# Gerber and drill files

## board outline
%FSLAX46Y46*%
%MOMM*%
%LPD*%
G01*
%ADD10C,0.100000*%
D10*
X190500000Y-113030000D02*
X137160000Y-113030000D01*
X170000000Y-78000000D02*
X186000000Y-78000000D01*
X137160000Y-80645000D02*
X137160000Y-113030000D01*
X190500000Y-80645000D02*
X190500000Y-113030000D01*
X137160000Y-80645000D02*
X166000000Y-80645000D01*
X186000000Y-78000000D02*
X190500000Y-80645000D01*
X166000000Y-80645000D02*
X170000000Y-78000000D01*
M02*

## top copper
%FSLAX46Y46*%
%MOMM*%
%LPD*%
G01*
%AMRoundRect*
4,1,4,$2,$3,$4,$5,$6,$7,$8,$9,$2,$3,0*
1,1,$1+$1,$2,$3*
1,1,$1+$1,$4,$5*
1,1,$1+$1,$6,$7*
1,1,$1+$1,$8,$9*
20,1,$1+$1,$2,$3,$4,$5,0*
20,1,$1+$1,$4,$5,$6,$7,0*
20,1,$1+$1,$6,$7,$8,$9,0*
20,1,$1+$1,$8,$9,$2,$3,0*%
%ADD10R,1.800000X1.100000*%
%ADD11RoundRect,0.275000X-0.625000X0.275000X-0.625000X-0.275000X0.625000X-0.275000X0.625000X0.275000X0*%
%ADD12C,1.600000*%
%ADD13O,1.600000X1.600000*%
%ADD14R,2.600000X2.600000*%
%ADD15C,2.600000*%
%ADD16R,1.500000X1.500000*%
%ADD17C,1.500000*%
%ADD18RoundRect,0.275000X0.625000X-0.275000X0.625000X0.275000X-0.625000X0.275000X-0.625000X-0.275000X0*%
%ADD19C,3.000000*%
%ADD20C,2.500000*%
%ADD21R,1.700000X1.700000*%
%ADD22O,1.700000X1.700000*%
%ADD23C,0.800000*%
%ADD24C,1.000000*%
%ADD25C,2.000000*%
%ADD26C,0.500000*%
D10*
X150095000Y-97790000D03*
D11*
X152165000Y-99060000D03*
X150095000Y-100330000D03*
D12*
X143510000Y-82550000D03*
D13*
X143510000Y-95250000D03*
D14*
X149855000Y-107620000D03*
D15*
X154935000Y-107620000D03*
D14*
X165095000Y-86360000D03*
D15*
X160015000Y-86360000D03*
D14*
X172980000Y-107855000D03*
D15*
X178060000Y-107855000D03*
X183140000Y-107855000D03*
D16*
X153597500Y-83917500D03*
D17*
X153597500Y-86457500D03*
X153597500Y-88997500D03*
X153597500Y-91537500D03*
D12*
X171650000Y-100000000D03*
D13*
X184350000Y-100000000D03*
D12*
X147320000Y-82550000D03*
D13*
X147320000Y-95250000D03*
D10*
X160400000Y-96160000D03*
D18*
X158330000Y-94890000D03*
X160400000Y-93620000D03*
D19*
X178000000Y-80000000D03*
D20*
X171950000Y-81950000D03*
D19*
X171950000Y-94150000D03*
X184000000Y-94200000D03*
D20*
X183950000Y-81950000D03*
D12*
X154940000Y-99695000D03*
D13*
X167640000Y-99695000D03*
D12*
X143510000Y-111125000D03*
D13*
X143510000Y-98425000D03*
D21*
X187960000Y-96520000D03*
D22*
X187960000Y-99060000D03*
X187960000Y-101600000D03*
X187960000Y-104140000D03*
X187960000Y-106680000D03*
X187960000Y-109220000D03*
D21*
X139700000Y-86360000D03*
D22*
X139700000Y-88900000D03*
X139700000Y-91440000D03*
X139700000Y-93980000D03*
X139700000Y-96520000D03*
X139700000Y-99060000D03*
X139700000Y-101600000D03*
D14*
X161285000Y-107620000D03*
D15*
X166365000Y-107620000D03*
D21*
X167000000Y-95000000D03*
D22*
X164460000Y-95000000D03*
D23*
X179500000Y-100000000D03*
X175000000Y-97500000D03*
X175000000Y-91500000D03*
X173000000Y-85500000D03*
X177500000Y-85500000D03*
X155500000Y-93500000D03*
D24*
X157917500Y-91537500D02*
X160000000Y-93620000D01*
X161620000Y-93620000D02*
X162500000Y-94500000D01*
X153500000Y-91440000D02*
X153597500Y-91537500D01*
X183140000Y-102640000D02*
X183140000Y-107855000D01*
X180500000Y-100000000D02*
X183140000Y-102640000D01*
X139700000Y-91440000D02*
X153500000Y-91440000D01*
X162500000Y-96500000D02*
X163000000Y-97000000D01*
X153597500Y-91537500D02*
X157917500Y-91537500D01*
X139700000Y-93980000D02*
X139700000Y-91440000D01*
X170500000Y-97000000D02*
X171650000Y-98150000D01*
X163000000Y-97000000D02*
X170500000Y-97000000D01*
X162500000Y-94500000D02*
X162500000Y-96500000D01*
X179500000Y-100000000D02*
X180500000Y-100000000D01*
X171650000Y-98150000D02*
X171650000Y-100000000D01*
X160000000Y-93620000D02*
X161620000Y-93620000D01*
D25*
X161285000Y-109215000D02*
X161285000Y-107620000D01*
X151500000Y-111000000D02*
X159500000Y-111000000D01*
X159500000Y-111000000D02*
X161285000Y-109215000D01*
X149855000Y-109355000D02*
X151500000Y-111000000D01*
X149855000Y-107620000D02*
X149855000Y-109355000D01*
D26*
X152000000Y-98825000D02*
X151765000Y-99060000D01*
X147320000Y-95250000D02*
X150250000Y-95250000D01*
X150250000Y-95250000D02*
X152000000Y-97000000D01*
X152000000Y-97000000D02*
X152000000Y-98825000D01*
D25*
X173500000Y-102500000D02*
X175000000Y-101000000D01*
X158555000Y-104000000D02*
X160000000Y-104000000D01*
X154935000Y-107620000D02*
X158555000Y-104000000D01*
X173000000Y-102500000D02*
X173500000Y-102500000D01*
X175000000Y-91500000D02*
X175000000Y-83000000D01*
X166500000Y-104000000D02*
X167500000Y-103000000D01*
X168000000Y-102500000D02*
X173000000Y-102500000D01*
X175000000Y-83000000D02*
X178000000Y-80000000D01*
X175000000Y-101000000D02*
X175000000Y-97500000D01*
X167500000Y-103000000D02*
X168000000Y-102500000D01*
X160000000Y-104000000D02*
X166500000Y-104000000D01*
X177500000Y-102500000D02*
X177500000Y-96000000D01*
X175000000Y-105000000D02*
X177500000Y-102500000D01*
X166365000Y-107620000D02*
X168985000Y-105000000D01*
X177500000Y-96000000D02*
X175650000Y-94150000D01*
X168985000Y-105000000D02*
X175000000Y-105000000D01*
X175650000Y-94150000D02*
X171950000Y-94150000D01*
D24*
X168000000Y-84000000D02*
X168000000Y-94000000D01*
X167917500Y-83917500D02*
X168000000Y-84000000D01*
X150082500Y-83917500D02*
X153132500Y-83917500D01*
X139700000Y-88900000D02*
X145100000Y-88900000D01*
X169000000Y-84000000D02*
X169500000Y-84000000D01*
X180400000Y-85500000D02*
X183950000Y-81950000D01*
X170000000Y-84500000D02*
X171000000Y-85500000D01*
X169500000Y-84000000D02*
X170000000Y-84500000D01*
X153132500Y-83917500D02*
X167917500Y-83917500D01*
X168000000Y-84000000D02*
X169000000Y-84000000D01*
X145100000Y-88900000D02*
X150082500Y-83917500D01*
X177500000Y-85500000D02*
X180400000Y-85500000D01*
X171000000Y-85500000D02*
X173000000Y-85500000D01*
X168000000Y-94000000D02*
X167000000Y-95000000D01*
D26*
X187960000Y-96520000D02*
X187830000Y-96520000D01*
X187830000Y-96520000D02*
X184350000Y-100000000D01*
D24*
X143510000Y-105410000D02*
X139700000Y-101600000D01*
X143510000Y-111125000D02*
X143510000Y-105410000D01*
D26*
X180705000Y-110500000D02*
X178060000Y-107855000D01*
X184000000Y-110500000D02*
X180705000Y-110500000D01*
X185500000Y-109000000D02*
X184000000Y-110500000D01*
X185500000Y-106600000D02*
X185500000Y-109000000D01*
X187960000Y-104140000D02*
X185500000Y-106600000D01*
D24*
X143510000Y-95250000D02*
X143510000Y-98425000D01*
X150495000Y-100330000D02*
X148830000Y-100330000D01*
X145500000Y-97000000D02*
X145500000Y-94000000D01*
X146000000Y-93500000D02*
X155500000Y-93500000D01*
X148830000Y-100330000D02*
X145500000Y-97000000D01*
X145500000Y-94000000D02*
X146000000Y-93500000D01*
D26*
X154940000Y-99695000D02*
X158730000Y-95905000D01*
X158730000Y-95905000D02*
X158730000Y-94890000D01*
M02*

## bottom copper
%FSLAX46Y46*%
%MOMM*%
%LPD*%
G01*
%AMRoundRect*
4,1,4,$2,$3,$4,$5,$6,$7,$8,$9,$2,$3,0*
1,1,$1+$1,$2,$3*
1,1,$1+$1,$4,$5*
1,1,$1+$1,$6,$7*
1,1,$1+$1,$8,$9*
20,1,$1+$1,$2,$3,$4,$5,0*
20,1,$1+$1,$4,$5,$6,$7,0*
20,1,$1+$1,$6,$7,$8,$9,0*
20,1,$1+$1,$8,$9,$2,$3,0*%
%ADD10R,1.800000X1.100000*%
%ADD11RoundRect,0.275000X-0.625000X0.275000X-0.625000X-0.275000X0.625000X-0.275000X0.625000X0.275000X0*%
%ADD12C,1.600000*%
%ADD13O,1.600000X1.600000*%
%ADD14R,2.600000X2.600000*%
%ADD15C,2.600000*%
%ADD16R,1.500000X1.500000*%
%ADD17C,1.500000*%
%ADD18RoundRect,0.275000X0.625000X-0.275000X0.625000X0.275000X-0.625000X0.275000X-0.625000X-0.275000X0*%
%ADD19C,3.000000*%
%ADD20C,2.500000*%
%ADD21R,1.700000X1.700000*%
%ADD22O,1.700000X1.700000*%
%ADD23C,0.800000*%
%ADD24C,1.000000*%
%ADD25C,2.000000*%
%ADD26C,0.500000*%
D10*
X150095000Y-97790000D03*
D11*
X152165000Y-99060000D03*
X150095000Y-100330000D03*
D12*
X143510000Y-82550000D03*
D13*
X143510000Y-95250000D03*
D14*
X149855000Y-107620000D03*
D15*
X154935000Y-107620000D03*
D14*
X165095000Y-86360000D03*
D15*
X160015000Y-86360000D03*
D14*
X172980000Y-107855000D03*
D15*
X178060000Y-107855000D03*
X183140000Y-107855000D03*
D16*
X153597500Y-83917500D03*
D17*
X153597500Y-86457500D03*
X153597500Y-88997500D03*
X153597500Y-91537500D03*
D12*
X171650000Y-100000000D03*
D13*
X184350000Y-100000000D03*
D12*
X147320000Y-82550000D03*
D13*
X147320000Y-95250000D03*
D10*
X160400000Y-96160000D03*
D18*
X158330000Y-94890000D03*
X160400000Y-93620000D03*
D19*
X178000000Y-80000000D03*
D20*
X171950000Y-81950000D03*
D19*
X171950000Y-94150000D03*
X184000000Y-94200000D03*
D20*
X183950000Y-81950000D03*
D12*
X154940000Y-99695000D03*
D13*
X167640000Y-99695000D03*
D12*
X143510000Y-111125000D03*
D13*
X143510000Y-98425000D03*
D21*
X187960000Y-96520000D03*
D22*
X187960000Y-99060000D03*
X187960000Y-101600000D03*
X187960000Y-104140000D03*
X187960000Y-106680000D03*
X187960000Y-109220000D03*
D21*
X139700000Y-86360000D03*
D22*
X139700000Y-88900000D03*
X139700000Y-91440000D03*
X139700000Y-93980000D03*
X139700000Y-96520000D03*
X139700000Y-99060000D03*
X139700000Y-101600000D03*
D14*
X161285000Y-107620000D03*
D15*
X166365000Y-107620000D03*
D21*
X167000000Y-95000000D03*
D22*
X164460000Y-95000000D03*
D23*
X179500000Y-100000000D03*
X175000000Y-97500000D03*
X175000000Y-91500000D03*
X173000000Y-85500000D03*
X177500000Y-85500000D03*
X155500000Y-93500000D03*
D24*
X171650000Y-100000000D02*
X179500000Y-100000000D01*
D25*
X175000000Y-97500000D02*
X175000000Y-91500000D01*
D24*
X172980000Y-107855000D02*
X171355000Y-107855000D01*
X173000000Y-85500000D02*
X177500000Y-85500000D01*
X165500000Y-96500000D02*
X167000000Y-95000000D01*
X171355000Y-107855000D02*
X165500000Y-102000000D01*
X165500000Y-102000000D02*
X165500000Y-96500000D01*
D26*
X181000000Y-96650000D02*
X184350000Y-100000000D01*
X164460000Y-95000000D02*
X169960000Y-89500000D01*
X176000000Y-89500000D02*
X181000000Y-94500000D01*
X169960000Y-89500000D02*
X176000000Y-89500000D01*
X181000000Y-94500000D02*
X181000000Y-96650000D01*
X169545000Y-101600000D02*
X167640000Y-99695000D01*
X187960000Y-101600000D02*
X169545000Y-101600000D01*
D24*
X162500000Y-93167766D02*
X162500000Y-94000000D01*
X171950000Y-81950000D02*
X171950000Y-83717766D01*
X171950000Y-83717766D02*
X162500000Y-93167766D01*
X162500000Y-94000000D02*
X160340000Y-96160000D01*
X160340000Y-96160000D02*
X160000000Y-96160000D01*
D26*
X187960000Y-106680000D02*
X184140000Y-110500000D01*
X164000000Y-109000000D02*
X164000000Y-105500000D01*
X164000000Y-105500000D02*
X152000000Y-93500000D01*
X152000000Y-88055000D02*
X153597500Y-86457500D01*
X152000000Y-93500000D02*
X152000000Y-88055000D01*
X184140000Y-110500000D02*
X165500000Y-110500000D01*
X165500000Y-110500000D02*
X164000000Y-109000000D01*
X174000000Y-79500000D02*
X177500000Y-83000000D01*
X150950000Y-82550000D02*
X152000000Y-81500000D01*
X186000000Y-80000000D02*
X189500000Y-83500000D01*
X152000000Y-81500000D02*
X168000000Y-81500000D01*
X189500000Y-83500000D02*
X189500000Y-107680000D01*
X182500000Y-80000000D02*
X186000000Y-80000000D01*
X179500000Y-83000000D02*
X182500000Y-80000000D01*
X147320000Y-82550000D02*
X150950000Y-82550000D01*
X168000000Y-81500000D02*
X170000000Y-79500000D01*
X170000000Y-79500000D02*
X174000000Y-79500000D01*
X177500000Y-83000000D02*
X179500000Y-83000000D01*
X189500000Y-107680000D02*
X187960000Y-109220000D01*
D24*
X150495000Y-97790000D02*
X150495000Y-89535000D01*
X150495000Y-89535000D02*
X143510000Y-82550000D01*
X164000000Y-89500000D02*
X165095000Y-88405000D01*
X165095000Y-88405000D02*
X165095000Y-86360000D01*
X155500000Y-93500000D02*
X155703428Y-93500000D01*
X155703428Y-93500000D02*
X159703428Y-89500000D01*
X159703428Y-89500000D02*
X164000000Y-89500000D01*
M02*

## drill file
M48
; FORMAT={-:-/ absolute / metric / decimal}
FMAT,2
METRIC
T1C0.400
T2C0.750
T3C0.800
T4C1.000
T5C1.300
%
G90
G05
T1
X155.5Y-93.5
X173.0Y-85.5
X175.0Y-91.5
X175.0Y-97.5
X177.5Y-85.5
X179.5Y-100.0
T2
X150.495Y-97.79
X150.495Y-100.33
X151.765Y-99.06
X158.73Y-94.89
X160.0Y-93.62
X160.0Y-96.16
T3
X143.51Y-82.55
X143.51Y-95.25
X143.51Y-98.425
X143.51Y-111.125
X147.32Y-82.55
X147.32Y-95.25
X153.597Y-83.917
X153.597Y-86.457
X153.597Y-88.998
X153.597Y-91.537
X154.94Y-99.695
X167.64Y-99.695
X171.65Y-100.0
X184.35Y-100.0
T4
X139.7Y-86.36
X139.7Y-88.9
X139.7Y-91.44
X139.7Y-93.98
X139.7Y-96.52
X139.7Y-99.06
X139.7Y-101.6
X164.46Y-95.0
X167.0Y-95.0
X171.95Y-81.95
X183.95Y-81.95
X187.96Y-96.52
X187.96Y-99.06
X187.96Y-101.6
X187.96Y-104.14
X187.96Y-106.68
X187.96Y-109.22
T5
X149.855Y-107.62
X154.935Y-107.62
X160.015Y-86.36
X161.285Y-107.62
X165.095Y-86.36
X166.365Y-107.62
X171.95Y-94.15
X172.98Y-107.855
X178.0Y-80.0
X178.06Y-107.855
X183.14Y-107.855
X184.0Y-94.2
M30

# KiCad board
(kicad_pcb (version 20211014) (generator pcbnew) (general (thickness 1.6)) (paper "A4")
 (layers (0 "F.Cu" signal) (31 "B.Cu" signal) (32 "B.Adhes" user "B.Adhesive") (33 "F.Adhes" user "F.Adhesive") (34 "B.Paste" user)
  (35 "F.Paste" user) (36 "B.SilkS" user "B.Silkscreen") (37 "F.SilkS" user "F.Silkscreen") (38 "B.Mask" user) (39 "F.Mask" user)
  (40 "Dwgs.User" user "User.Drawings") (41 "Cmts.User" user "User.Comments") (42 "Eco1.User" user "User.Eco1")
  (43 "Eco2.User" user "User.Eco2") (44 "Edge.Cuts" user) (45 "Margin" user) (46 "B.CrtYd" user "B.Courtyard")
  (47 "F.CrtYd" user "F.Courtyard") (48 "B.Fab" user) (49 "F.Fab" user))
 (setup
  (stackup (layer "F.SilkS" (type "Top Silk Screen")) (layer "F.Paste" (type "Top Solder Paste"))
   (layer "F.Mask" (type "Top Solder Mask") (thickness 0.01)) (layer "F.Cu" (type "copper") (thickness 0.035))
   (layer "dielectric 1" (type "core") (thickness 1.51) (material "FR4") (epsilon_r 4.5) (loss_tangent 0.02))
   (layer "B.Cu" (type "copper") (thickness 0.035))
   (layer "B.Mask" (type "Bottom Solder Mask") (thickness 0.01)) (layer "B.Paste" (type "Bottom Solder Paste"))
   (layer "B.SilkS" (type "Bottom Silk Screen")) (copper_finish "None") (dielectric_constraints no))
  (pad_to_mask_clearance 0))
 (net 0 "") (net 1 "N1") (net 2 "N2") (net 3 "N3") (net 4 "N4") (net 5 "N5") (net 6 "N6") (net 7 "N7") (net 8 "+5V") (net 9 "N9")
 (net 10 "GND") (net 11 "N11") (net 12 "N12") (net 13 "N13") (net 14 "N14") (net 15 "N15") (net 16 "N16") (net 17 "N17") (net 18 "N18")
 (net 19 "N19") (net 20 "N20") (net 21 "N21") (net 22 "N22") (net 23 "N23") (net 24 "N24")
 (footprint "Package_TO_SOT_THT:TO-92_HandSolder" (layer "F.Cu") (at 150.495 97.79 -90)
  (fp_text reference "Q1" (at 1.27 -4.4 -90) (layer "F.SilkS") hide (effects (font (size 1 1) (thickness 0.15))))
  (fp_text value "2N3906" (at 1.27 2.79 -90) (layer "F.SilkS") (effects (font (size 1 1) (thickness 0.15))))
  (pad "1" thru_hole rect (at 0 0 270) (size 1.1 1.8) (drill 0.75 (offset 0 0.4)) (layers *.Cu *.Mask) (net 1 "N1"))
  (pad "2" thru_hole roundrect (at 1.27 -1.27 270) (size 1.1 1.8) (drill 0.75 (offset 0 -0.4)) (layers *.Cu *.Mask) (roundrect_rratio 0.25)
   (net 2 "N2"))
  (pad "3" thru_hole roundrect (at 2.54 0 270) (size 1.1 1.8) (drill 0.75 (offset 0 0.4)) (layers *.Cu *.Mask) (roundrect_rratio 0.25)
   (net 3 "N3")))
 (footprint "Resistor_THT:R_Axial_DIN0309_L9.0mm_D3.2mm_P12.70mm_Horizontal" (layer "F.Cu") (at 143.51 82.55 -90)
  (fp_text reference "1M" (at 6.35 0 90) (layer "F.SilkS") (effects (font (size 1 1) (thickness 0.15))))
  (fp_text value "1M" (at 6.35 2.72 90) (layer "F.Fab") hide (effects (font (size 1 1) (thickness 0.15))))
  (pad "1" thru_hole circle (at 0 0 270) (size 1.6 1.6) (drill 0.8) (layers *.Cu *.Mask) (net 1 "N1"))
  (pad "2" thru_hole oval (at 12.7 0 270) (size 1.6 1.6) (drill 0.8) (layers *.Cu *.Mask) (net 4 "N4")))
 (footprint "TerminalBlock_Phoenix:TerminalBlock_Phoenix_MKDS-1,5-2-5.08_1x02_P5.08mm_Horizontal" (layer "F.Cu") (at 149.855 107.62)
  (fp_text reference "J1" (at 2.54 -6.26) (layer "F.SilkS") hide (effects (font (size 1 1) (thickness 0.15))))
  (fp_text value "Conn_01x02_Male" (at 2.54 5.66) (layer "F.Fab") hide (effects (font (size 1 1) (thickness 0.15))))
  (pad "1" thru_hole rect (at 0 0) (size 2.6 2.6) (drill 1.3) (layers *.Cu *.Mask) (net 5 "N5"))
  (pad "2" thru_hole circle (at 5.08 0) (size 2.6 2.6) (drill 1.3) (layers *.Cu *.Mask) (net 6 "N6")))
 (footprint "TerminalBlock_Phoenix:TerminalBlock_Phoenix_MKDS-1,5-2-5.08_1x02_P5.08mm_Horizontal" (layer "F.Cu") (at 165.095 86.36 180)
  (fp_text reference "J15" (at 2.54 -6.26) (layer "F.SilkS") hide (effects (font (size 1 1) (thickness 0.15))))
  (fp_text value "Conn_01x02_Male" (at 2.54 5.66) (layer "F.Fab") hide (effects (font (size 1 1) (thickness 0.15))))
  (pad "1" thru_hole rect (at 0 0 180) (size 2.6 2.6) (drill 1.3) (layers *.Cu *.Mask) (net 3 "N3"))
  (pad "2" thru_hole circle (at 5.08 0 180) (size 2.6 2.6) (drill 1.3) (layers *.Cu *.Mask) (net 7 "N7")))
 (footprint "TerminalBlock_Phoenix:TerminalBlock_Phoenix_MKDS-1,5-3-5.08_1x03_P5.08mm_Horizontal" (layer "F.Cu") (at 172.98 107.855)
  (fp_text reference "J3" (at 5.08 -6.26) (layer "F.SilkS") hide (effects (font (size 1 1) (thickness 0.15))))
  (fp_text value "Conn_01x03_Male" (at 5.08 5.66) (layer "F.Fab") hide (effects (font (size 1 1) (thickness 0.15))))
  (pad "1" thru_hole rect (at 0 0) (size 2.6 2.6) (drill 1.3) (layers *.Cu *.Mask) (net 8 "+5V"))
  (pad "2" thru_hole circle (at 5.08 0) (size 2.6 2.6) (drill 1.3) (layers *.Cu *.Mask) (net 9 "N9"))
  (pad "3" thru_hole circle (at 10.16 0) (size 2.6 2.6) (drill 1.3) (layers *.Cu *.Mask) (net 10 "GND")))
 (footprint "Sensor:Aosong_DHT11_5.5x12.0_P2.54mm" (layer "F.Cu") (at 153.5975 83.9175)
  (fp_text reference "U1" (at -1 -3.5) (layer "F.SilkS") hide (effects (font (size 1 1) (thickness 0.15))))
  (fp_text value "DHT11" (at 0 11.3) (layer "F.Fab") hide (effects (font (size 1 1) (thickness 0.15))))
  (pad "1" thru_hole rect (at 0 0) (size 1.5 1.5) (drill 0.8) (layers *.Cu *.Mask) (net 8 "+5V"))
  (pad "2" thru_hole circle (at 0 2.54) (size 1.5 1.5) (drill 0.8) (layers *.Cu *.Mask) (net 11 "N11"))
  (pad "3" thru_hole circle (at 0 5.08) (size 1.5 1.5) (drill 0.8) (layers *.Cu *.Mask) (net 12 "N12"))
  (pad "4" thru_hole circle (at 0 7.62) (size 1.5 1.5) (drill 0.8) (layers *.Cu *.Mask) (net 10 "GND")))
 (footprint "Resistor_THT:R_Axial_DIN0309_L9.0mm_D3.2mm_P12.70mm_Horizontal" (layer "F.Cu") (at 171.65 100)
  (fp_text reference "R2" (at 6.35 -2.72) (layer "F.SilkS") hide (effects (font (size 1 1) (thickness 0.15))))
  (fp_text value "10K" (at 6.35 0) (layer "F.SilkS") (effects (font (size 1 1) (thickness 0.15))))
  (pad "1" thru_hole circle (at 0 0) (size 1.6 1.6) (drill 0.8) (layers *.Cu *.Mask) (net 10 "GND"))
  (pad "2" thru_hole oval (at 12.7 0) (size 1.6 1.6) (drill 0.8) (layers *.Cu *.Mask) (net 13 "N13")))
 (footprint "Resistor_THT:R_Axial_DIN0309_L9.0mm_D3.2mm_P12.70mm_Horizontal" (layer "F.Cu") (at 147.32 82.55 -90)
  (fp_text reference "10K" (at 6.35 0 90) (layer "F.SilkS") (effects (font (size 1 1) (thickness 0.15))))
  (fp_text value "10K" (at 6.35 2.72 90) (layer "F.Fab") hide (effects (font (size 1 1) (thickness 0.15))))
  (pad "1" thru_hole circle (at 0 0 270) (size 1.6 1.6) (drill 0.8) (layers *.Cu *.Mask) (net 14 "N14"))
  (pad "2" thru_hole oval (at 12.7 0 270) (size 1.6 1.6) (drill 0.8) (layers *.Cu *.Mask) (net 2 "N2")))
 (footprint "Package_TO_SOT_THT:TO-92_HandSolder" (layer "F.Cu") (at 160 96.16 90)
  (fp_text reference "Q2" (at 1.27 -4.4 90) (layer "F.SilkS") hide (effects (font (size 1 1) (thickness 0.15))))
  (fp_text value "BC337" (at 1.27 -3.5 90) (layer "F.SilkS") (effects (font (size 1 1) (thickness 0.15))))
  (pad "1" thru_hole rect (at 0 0 90) (size 1.1 1.8) (drill 0.75 (offset 0 0.4)) (layers *.Cu *.Mask) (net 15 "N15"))
  (pad "2" thru_hole roundrect (at 1.27 -1.27 90) (size 1.1 1.8) (drill 0.75 (offset 0 -0.4)) (layers *.Cu *.Mask) (roundrect_rratio 0.25)
   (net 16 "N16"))
  (pad "3" thru_hole roundrect (at 2.54 0 90) (size 1.1 1.8) (drill 0.75 (offset 0 0.4)) (layers *.Cu *.Mask) (roundrect_rratio 0.25)
   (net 10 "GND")))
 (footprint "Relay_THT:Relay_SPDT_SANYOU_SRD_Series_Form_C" (layer "F.Cu") (at 178 80 -90)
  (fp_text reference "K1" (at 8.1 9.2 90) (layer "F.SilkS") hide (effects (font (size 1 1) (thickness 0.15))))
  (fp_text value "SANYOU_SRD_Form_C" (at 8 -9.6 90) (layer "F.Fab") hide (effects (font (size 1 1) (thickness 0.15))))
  (pad "1" thru_hole circle (at 0 0) (size 3 3) (drill 1.3) (layers *.Cu *.Mask) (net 6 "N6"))
  (pad "2" thru_hole circle (at 1.95 6.05) (size 2.5 2.5) (drill 1) (layers *.Cu *.Mask) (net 15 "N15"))
  (pad "3" thru_hole circle (at 14.15 6.05) (size 3 3) (drill 1.3) (layers *.Cu *.Mask) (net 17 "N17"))
  (pad "4" thru_hole circle (at 14.2 -6) (size 3 3) (drill 1.3) (layers *.Cu *.Mask) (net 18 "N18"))
  (pad "5" thru_hole circle (at 1.95 -5.95) (size 2.5 2.5) (drill 1) (layers *.Cu *.Mask) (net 8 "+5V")))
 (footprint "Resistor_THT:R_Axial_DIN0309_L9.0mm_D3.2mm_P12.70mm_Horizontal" (layer "F.Cu") (at 154.94 99.695)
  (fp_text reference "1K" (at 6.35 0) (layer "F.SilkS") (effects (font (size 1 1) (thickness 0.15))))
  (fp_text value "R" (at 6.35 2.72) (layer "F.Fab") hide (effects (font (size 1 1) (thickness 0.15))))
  (pad "1" thru_hole circle (at 0 0) (size 1.6 1.6) (drill 0.8) (layers *.Cu *.Mask) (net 16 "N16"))
  (pad "2" thru_hole oval (at 12.7 0) (size 1.6 1.6) (drill 0.8) (layers *.Cu *.Mask) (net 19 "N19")))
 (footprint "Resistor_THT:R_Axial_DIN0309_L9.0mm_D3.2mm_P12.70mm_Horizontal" (layer "F.Cu") (at 143.51 111.125 90)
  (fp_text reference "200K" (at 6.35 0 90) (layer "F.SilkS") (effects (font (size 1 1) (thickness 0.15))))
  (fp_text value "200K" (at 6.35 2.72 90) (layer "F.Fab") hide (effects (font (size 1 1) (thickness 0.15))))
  (pad "1" thru_hole circle (at 0 0 90) (size 1.6 1.6) (drill 0.8) (layers *.Cu *.Mask) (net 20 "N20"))
  (pad "2" thru_hole oval (at 12.7 0 90) (size 1.6 1.6) (drill 0.8) (layers *.Cu *.Mask) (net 4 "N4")))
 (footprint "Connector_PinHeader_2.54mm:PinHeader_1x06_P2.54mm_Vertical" (layer "F.Cu") (at 187.96 96.52)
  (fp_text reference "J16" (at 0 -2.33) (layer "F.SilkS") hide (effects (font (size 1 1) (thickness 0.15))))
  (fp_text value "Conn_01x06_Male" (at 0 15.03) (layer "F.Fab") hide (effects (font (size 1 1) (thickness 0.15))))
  (pad "1" thru_hole rect (at 0 0) (size 1.7 1.7) (drill 1) (layers *.Cu *.Mask) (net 13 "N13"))
  (pad "2" thru_hole oval (at 0 2.54) (size 1.7 1.7) (drill 1) (layers *.Cu *.Mask) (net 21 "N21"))
  (pad "3" thru_hole oval (at 0 5.08) (size 1.7 1.7) (drill 1) (layers *.Cu *.Mask) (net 19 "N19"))
  (pad "4" thru_hole oval (at 0 7.62) (size 1.7 1.7) (drill 1) (layers *.Cu *.Mask) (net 9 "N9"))
  (pad "5" thru_hole oval (at 0 10.16) (size 1.7 1.7) (drill 1) (layers *.Cu *.Mask) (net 11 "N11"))
  (pad "6" thru_hole oval (at 0 12.7) (size 1.7 1.7) (drill 1) (layers *.Cu *.Mask) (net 14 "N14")))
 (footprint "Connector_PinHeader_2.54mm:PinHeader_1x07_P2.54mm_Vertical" (layer "F.Cu") (at 139.7 86.36)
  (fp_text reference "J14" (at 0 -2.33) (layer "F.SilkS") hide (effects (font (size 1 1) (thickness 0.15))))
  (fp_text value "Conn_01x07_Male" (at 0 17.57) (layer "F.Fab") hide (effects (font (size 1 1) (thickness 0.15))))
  (pad "1" thru_hole rect (at 0 0) (size 1.7 1.7) (drill 1) (layers *.Cu *.Mask) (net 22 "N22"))
  (pad "2" thru_hole oval (at 0 2.54) (size 1.7 1.7) (drill 1) (layers *.Cu *.Mask) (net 8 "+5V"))
  (pad "3" thru_hole oval (at 0 5.08) (size 1.7 1.7) (drill 1) (layers *.Cu *.Mask) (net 10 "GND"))
  (pad "4" thru_hole oval (at 0 7.62) (size 1.7 1.7) (drill 1) (layers *.Cu *.Mask) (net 10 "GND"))
  (pad "5" thru_hole oval (at 0 10.16) (size 1.7 1.7) (drill 1) (layers *.Cu *.Mask) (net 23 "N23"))
  (pad "6" thru_hole oval (at 0 12.7) (size 1.7 1.7) (drill 1) (layers *.Cu *.Mask) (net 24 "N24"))
  (pad "7" thru_hole oval (at 0 15.24) (size 1.7 1.7) (drill 1) (layers *.Cu *.Mask) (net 20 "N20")))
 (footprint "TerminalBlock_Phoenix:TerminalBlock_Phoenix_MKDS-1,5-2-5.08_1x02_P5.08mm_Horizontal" (layer "F.Cu") (at 161.285 107.62)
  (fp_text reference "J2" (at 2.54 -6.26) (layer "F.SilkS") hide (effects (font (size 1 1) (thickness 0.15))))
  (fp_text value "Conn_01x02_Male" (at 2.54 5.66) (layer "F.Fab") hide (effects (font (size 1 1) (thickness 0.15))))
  (pad "1" thru_hole rect (at 0 0) (size 2.6 2.6) (drill 1.3) (layers *.Cu *.Mask) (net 5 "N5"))
  (pad "2" thru_hole circle (at 5.08 0) (size 2.6 2.6) (drill 1.3) (layers *.Cu *.Mask) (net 17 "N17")))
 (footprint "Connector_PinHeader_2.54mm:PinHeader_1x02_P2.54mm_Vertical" (layer "F.Cu") (at 167 95 -90)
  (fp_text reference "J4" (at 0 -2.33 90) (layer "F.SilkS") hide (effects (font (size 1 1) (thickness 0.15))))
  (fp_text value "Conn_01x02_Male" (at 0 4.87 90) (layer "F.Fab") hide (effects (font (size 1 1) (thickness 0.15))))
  (pad "1" thru_hole rect (at 0 0 270) (size 1.7 1.7) (drill 1) (layers *.Cu *.Mask) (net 8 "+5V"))
  (pad "2" thru_hole oval (at 0 2.54 270) (size 1.7 1.7) (drill 1) (layers *.Cu *.Mask) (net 13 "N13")))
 (gr_line (start 190.5 113.03) (end 137.16 113.03) (layer "Edge.Cuts") (width 0.1))
 (gr_line (start 170 78) (end 186 78) (layer "Edge.Cuts") (width 0.1))
 (gr_line (start 137.16 80.645) (end 137.16 113.03) (layer "Edge.Cuts") (width 0.1))
 (gr_line (start 190.5 80.645) (end 190.5 113.03) (layer "Edge.Cuts") (width 0.1))
 (gr_line (start 137.16 80.645) (end 166 80.645) (layer "Edge.Cuts") (width 0.1))
 (gr_line (start 186 78) (end 190.5 80.645) (layer "Edge.Cuts") (width 0.1))
 (gr_line (start 166 80.645) (end 170 78) (layer "Edge.Cuts") (width 0.1))
 (segment (start 157.9175 91.5375) (end 160 93.62) (width 1) (layer "F.Cu") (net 10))
 (segment (start 161.62 93.62) (end 162.5 94.5) (width 1) (layer "F.Cu") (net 10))
 (segment (start 153.5 91.44) (end 153.5975 91.5375) (width 1) (layer "F.Cu") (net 10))
 (segment (start 183.14 102.64) (end 183.14 107.855) (width 1) (layer "F.Cu") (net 10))
 (segment (start 180.5 100) (end 183.14 102.64) (width 1) (layer "F.Cu") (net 10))
 (segment (start 139.7 91.44) (end 153.5 91.44) (width 1) (layer "F.Cu") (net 10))
 (segment (start 162.5 96.5) (end 163 97) (width 1) (layer "F.Cu") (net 10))
 (segment (start 153.5975 91.5375) (end 157.9175 91.5375) (width 1) (layer "F.Cu") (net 10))
 (segment (start 139.7 93.98) (end 139.7 91.44) (width 1) (layer "F.Cu") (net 10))
 (segment (start 170.5 97) (end 171.65 98.15) (width 1) (layer "F.Cu") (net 10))
 (segment (start 163 97) (end 170.5 97) (width 1) (layer "F.Cu") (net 10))
 (segment (start 162.5 94.5) (end 162.5 96.5) (width 1) (layer "F.Cu") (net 10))
 (segment (start 179.5 100) (end 180.5 100) (width 1) (layer "F.Cu") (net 10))
 (segment (start 171.65 98.15) (end 171.65 100) (width 1) (layer "F.Cu") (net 10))
 (segment (start 160 93.62) (end 161.62 93.62) (width 1) (layer "F.Cu") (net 10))
 (via (at 179.5 100) (size 0.8) (drill 0.4) (layers "F.Cu" "B.Cu") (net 10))
 (segment (start 171.65 100) (end 179.5 100) (width 1) (layer "B.Cu") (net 10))
 (segment (start 161.285 109.215) (end 161.285 107.62) (width 2) (layer "F.Cu") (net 5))
 (segment (start 151.5 111) (end 159.5 111) (width 2) (layer "F.Cu") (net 5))
 (segment (start 159.5 111) (end 161.285 109.215) (width 2) (layer "F.Cu") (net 5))
 (segment (start 149.855 109.355) (end 151.5 111) (width 2) (layer "F.Cu") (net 5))
 (segment (start 149.855 107.62) (end 149.855 109.355) (width 2) (layer "F.Cu") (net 5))
 (segment (start 152 98.825) (end 151.765 99.06) (width 0.5) (layer "F.Cu") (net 2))
 (segment (start 147.32 95.25) (end 150.25 95.25) (width 0.5) (layer "F.Cu") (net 2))
 (segment (start 150.25 95.25) (end 152 97) (width 0.5) (layer "F.Cu") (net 2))
 (segment (start 152 97) (end 152 98.825) (width 0.5) (layer "F.Cu") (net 2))
 (segment (start 173.5 102.5) (end 175 101) (width 2) (layer "F.Cu") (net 6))
 (segment (start 158.555 104) (end 160 104) (width 2) (layer "F.Cu") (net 6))
 (segment (start 154.935 107.62) (end 158.555 104) (width 2) (layer "F.Cu") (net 6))
 (segment (start 173 102.5) (end 173.5 102.5) (width 2) (layer "F.Cu") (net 6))
 (segment (start 175 91.5) (end 175 83) (width 2) (layer "F.Cu") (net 6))
 (segment (start 166.5 104) (end 167.5 103) (width 2) (layer "F.Cu") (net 6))
 (segment (start 168 102.5) (end 173 102.5) (width 2) (layer "F.Cu") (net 6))
 (segment (start 175 83) (end 178 80) (width 2) (layer "F.Cu") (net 6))
 (segment (start 175 101) (end 175 97.5) (width 2) (layer "F.Cu") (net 6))
 (segment (start 167.5 103) (end 168 102.5) (width 2) (layer "F.Cu") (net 6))
 (segment (start 160 104) (end 166.5 104) (width 2) (layer "F.Cu") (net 6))
 (via (at 175 97.5) (size 0.8) (drill 0.4) (layers "F.Cu" "B.Cu") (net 6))
 (via (at 175 91.5) (size 0.8) (drill 0.4) (layers "F.Cu" "B.Cu") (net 6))
 (segment (start 175 97.5) (end 175 91.5) (width 2) (layer "B.Cu") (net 6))
 (segment (start 177.5 102.5) (end 177.5 96) (width 2) (layer "F.Cu") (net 17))
 (segment (start 175 105) (end 177.5 102.5) (width 2) (layer "F.Cu") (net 17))
 (segment (start 166.365 107.62) (end 168.985 105) (width 2) (layer "F.Cu") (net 17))
 (segment (start 177.5 96) (end 175.65 94.15) (width 2) (layer "F.Cu") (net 17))
 (segment (start 168.985 105) (end 175 105) (width 2) (layer "F.Cu") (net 17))
 (segment (start 175.65 94.15) (end 171.95 94.15) (width 2) (layer "F.Cu") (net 17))
 (segment (start 168 84) (end 168 94) (width 1) (layer "F.Cu") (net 8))
 (segment (start 167.9175 83.9175) (end 168 84) (width 1) (layer "F.Cu") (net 8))
 (segment (start 150.0825 83.9175) (end 153.1325 83.9175) (width 1) (layer "F.Cu") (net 8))
 (segment (start 139.7 88.9) (end 145.1 88.9) (width 1) (layer "F.Cu") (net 8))
 (segment (start 169 84) (end 169.5 84) (width 1) (layer "F.Cu") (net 8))
 (segment (start 180.4 85.5) (end 183.95 81.95) (width 1) (layer "F.Cu") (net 8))
 (segment (start 170 84.5) (end 171 85.5) (width 1) (layer "F.Cu") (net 8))
 (segment (start 169.5 84) (end 170 84.5) (width 1) (layer "F.Cu") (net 8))
 (segment (start 153.1325 83.9175) (end 167.9175 83.9175) (width 1) (layer "F.Cu") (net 8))
 (segment (start 168 84) (end 169 84) (width 1) (layer "F.Cu") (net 8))
 (segment (start 145.1 88.9) (end 150.0825 83.9175) (width 1) (layer "F.Cu") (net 8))
 (segment (start 177.5 85.5) (end 180.4 85.5) (width 1) (layer "F.Cu") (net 8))
 (segment (start 171 85.5) (end 173 85.5) (width 1) (layer "F.Cu") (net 8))
 (segment (start 168 94) (end 167 95) (width 1) (layer "F.Cu") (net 8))
 (via (at 173 85.5) (size 0.8) (drill 0.4) (layers "F.Cu" "B.Cu") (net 8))
 (via (at 177.5 85.5) (size 0.8) (drill 0.4) (layers "F.Cu" "B.Cu") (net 8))
 (segment (start 172.98 107.855) (end 171.355 107.855) (width 1) (layer "B.Cu") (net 8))
 (segment (start 173 85.5) (end 177.5 85.5) (width 1) (layer "B.Cu") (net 8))
 (segment (start 165.5 96.5) (end 167 95) (width 1) (layer "B.Cu") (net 8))
 (segment (start 171.355 107.855) (end 165.5 102) (width 1) (layer "B.Cu") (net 8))
 (segment (start 165.5 102) (end 165.5 96.5) (width 1) (layer "B.Cu") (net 8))
 (segment (start 187.96 96.52) (end 187.83 96.52) (width 0.5) (layer "F.Cu") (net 13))
 (segment (start 187.83 96.52) (end 184.35 100) (width 0.5) (layer "F.Cu") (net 13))
 (segment (start 181 96.65) (end 184.35 100) (width 0.5) (layer "B.Cu") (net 13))
 (segment (start 164.46 95) (end 169.96 89.5) (width 0.5) (layer "B.Cu") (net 13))
 (segment (start 176 89.5) (end 181 94.5) (width 0.5) (layer "B.Cu") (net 13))
 (segment (start 169.96 89.5) (end 176 89.5) (width 0.5) (layer "B.Cu") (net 13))
 (segment (start 181 94.5) (end 181 96.65) (width 0.5) (layer "B.Cu") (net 13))
 (segment (start 169.545 101.6) (end 167.64 99.695) (width 0.5) (layer "B.Cu") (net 19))
 (segment (start 187.96 101.6) (end 169.545 101.6) (width 0.5) (layer "B.Cu") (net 19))
 (segment (start 162.5 93.167766) (end 162.5 94) (width 1) (layer "B.Cu") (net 15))
 (segment (start 171.95 81.95) (end 171.95 83.717766) (width 1) (layer "B.Cu") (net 15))
 (segment (start 171.95 83.717766) (end 162.5 93.167766) (width 1) (layer "B.Cu") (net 15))
 (segment (start 162.5 94) (end 160.34 96.16) (width 1) (layer "B.Cu") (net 15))
 (segment (start 160.34 96.16) (end 160 96.16) (width 1) (layer "B.Cu") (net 15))
 (segment (start 143.51 105.41) (end 139.7 101.6) (width 1) (layer "F.Cu") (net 20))
 (segment (start 143.51 111.125) (end 143.51 105.41) (width 1) (layer "F.Cu") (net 20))
 (segment (start 180.705 110.5) (end 178.06 107.855) (width 0.5) (layer "F.Cu") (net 9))
 (segment (start 184 110.5) (end 180.705 110.5) (width 0.5) (layer "F.Cu") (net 9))
 (segment (start 185.5 109) (end 184 110.5) (width 0.5) (layer "F.Cu") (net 9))
 (segment (start 185.5 106.6) (end 185.5 109) (width 0.5) (layer "F.Cu") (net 9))
 (segment (start 187.96 104.14) (end 185.5 106.6) (width 0.5) (layer "F.Cu") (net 9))
 (segment (start 187.96 106.68) (end 184.14 110.5) (width 0.5) (layer "B.Cu") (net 11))
 (segment (start 164 109) (end 164 105.5) (width 0.5) (layer "B.Cu") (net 11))
 (segment (start 164 105.5) (end 152 93.5) (width 0.5) (layer "B.Cu") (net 11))
 (segment (start 152 88.055) (end 153.5975 86.4575) (width 0.5) (layer "B.Cu") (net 11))
 (segment (start 152 93.5) (end 152 88.055) (width 0.5) (layer "B.Cu") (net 11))
 (segment (start 184.14 110.5) (end 165.5 110.5) (width 0.5) (layer "B.Cu") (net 11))
 (segment (start 165.5 110.5) (end 164 109) (width 0.5) (layer "B.Cu") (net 11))
 (segment (start 174 79.5) (end 177.5 83) (width 0.5) (layer "B.Cu") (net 14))
 (segment (start 150.95 82.55) (end 152 81.5) (width 0.5) (layer "B.Cu") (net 14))
 (segment (start 186 80) (end 189.5 83.5) (width 0.5) (layer "B.Cu") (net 14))
 (segment (start 152 81.5) (end 168 81.5) (width 0.5) (layer "B.Cu") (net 14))
 (segment (start 189.5 83.5) (end 189.5 107.68) (width 0.5) (layer "B.Cu") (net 14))
 (segment (start 182.5 80) (end 186 80) (width 0.5) (layer "B.Cu") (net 14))
 (segment (start 179.5 83) (end 182.5 80) (width 0.5) (layer "B.Cu") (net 14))
 (segment (start 147.32 82.55) (end 150.95 82.55) (width 0.5) (layer "B.Cu") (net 14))
 (segment (start 168 81.5) (end 170 79.5) (width 0.5) (layer "B.Cu") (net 14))
 (segment (start 170 79.5) (end 174 79.5) (width 0.5) (layer "B.Cu") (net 14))
 (segment (start 177.5 83) (end 179.5 83) (width 0.5) (layer "B.Cu") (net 14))
 (segment (start 189.5 107.68) (end 187.96 109.22) (width 0.5) (layer "B.Cu") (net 14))
 (segment (start 150.495 97.79) (end 150.495 89.535) (width 1) (layer "B.Cu") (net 1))
 (segment (start 150.495 89.535) (end 143.51 82.55) (width 1) (layer "B.Cu") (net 1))
 (segment (start 143.51 95.25) (end 143.51 98.425) (width 1) (layer "F.Cu") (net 4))
 (segment (start 150.495 100.33) (end 148.83 100.33) (width 1) (layer "F.Cu") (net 3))
 (segment (start 145.5 97) (end 145.5 94) (width 1) (layer "F.Cu") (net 3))
 (segment (start 146 93.5) (end 155.5 93.5) (width 1) (layer "F.Cu") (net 3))
 (segment (start 148.83 100.33) (end 145.5 97) (width 1) (layer "F.Cu") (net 3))
 (segment (start 145.5 94) (end 146 93.5) (width 1) (layer "F.Cu") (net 3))
 (via (at 155.5 93.5) (size 0.8) (drill 0.4) (layers "F.Cu" "B.Cu") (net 3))
 (segment (start 164 89.5) (end 165.095 88.405) (width 1) (layer "B.Cu") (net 3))
 (segment (start 165.095 88.405) (end 165.095 86.36) (width 1) (layer "B.Cu") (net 3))
 (segment (start 155.5 93.5) (end 155.703428 93.5) (width 1) (layer "B.Cu") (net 3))
 (segment (start 155.703428 93.5) (end 159.703428 89.5) (width 1) (layer "B.Cu") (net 3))
 (segment (start 159.703428 89.5) (end 164 89.5) (width 1) (layer "B.Cu") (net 3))
 (segment (start 154.94 99.695) (end 158.73 95.905) (width 0.5) (layer "F.Cu") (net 16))
 (segment (start 158.73 95.905) (end 158.73 94.89) (width 0.5) (layer "F.Cu") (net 16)))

